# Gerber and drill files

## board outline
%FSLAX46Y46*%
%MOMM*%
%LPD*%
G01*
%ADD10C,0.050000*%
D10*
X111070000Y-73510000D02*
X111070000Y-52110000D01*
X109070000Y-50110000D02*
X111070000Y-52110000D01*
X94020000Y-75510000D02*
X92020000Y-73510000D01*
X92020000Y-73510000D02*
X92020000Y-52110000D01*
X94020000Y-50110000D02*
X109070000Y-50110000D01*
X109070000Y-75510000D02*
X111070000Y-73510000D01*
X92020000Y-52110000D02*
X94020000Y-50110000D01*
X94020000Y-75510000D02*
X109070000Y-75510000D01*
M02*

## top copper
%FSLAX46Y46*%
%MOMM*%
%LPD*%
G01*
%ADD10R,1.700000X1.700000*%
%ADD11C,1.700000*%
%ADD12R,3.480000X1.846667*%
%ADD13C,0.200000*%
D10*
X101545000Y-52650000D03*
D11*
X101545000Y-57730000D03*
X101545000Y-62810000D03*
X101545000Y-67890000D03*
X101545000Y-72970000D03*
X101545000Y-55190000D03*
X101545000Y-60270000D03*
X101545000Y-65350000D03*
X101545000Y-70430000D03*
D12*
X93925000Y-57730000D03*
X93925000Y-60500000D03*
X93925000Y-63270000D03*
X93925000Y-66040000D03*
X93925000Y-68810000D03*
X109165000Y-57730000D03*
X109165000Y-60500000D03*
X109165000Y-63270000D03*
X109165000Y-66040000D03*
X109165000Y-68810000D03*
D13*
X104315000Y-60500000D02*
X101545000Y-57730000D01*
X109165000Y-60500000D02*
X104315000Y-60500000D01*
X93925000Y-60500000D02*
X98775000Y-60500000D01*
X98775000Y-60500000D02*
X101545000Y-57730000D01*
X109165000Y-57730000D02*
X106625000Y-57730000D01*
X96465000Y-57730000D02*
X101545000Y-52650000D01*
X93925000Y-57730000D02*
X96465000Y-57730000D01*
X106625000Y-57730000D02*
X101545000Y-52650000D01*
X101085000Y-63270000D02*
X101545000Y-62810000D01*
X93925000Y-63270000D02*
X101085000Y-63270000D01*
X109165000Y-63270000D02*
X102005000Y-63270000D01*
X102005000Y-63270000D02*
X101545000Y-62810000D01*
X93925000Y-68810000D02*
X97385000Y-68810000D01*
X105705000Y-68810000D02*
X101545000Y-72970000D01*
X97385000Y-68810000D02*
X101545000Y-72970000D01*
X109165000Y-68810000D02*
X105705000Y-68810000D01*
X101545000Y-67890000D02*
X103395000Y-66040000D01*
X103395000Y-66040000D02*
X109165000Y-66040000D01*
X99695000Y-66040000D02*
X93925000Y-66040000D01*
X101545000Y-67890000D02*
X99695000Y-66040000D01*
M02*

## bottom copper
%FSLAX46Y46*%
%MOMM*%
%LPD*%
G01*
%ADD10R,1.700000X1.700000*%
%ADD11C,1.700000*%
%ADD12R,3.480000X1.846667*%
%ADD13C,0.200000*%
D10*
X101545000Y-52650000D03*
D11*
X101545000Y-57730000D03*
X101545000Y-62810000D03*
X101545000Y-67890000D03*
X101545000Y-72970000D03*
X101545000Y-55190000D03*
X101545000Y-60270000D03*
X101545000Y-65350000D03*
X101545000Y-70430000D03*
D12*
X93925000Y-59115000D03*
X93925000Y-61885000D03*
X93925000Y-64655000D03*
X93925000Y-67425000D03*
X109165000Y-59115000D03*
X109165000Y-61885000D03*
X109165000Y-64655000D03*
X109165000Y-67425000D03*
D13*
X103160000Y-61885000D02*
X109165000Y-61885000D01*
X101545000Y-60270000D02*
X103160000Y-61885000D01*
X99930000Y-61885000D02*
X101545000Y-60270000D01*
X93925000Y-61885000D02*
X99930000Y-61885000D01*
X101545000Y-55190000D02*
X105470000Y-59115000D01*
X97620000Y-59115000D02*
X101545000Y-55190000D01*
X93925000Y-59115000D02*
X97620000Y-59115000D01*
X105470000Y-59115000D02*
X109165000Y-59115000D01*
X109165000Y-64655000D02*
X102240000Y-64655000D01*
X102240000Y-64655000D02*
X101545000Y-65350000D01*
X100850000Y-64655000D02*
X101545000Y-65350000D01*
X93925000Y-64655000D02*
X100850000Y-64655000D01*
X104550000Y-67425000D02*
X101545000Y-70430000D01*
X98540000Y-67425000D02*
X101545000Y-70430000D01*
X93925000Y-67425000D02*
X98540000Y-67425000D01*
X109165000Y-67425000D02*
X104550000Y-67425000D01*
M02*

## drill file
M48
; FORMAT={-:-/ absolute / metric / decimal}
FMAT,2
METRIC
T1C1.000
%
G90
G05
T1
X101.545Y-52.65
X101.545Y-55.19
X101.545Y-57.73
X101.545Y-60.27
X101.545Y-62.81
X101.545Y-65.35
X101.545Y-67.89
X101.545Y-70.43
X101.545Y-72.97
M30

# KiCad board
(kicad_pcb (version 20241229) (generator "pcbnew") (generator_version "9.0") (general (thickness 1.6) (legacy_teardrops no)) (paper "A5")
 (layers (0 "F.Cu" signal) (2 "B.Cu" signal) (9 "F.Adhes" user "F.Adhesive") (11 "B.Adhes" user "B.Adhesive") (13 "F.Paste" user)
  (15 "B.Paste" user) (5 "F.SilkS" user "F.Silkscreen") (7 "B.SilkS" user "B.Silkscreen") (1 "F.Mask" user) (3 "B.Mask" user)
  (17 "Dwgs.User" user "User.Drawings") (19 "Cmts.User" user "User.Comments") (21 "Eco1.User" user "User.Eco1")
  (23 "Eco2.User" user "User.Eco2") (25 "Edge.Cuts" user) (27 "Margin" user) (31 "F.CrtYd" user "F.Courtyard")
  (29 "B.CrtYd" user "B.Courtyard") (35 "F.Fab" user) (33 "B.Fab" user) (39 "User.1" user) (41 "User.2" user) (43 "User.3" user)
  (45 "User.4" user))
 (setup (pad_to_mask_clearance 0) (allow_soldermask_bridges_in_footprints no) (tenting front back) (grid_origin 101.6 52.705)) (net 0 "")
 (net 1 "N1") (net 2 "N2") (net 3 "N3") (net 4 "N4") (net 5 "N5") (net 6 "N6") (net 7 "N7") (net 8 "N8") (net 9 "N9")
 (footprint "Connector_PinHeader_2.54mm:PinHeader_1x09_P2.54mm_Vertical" (layer "F.Cu") (at 101.545 72.97 180)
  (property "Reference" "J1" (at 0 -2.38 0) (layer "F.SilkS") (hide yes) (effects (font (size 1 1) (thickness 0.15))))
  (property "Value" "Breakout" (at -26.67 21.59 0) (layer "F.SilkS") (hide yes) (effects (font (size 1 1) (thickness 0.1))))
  (pad "1" thru_hole rect (at 0 20.32 180) (size 1.7 1.7) (drill 1) (layers "*.Cu" "*.Mask") (remove_unused_layers no) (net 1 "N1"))
  (pad "2" thru_hole circle (at 0 15.24 180) (size 1.7 1.7) (drill 1) (layers "*.Cu" "*.Mask") (remove_unused_layers no) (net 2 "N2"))
  (pad "3" thru_hole circle (at 0 10.16 180) (size 1.7 1.7) (drill 1) (layers "*.Cu" "*.Mask") (remove_unused_layers no) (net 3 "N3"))
  (pad "4" thru_hole circle (at 0 5.08 180) (size 1.7 1.7) (drill 1) (layers "*.Cu" "*.Mask") (remove_unused_layers no) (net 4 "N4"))
  (pad "5" thru_hole circle (at 0 0 180) (size 1.7 1.7) (drill 1) (layers "*.Cu" "*.Mask") (remove_unused_layers no) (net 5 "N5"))
  (pad "6" thru_hole circle (at 0 17.78 180) (size 1.7 1.7) (drill 1) (layers "*.Cu" "*.Mask") (remove_unused_layers no) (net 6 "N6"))
  (pad "7" thru_hole circle (at 0 12.7 180) (size 1.7 1.7) (drill 1) (layers "*.Cu" "*.Mask") (remove_unused_layers no) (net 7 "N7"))
  (pad "8" thru_hole circle (at 0 7.62 180) (size 1.7 1.7) (drill 1) (layers "*.Cu" "*.Mask") (remove_unused_layers no) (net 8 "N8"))
  (pad "9" thru_hole circle (at 0 2.54 180) (size 1.7 1.7) (drill 1) (layers "*.Cu" "*.Mask") (remove_unused_layers no) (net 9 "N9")))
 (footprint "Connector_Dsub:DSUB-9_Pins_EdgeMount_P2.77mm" (layer "F.Cu") (at 93.925 63.27 -90)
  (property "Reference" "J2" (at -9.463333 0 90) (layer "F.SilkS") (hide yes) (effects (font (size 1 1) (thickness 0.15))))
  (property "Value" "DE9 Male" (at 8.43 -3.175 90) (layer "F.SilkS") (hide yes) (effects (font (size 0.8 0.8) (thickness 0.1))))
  (pad "1" smd rect (at -5.54 0 270) (size 1.846667 3.48) (layers "F.Cu" "F.Mask" "F.Paste") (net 1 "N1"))
  (pad "2" smd rect (at -2.77 0 270) (size 1.846667 3.48) (layers "F.Cu" "F.Mask" "F.Paste") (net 2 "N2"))
  (pad "3" smd rect (at 0 0 270) (size 1.846667 3.48) (layers "F.Cu" "F.Mask" "F.Paste") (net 3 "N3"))
  (pad "4" smd rect (at 2.77 0 270) (size 1.846667 3.48) (layers "F.Cu" "F.Mask" "F.Paste") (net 4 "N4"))
  (pad "5" smd rect (at 5.54 0 270) (size 1.846667 3.48) (layers "F.Cu" "F.Mask" "F.Paste") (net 5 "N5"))
  (pad "6" smd rect (at -4.155 0 270) (size 1.846667 3.48) (layers "B.Cu" "B.Mask" "B.Paste") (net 6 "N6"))
  (pad "7" smd rect (at -1.385 0 270) (size 1.846667 3.48) (layers "B.Cu" "B.Mask" "B.Paste") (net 7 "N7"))
  (pad "8" smd rect (at 1.385 0 270) (size 1.846667 3.48) (layers "B.Cu" "B.Mask" "B.Paste") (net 8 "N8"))
  (pad "9" smd rect (at 4.155 0 270) (size 1.846667 3.48) (layers "B.Cu" "B.Mask" "B.Paste") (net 9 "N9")))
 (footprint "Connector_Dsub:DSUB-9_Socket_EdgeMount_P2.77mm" (layer "F.Cu") (at 109.165 63.27 90)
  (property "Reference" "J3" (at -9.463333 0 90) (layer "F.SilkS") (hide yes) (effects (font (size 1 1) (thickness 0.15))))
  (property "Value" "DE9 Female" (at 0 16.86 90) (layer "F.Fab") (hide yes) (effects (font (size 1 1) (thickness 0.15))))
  (pad "1" smd rect (at 5.54 0 90) (size 1.846667 3.48) (layers "F.Cu" "F.Mask" "F.Paste") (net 1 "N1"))
  (pad "2" smd rect (at 2.77 0 90) (size 1.846667 3.48) (layers "F.Cu" "F.Mask" "F.Paste") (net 2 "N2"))
  (pad "3" smd rect (at 0 0 90) (size 1.846667 3.48) (layers "F.Cu" "F.Mask" "F.Paste") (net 3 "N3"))
  (pad "4" smd rect (at -2.77 0 90) (size 1.846667 3.48) (layers "F.Cu" "F.Mask" "F.Paste") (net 4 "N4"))
  (pad "5" smd rect (at -5.54 0 90) (size 1.846667 3.48) (layers "F.Cu" "F.Mask" "F.Paste") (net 5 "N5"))
  (pad "6" smd rect (at 4.155 0 90) (size 1.846667 3.48) (layers "B.Cu" "B.Mask" "B.Paste") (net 6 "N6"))
  (pad "7" smd rect (at 1.385 0 90) (size 1.846667 3.48) (layers "B.Cu" "B.Mask" "B.Paste") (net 7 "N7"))
  (pad "8" smd rect (at -1.385 0 90) (size 1.846667 3.48) (layers "B.Cu" "B.Mask" "B.Paste") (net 8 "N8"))
  (pad "9" smd rect (at -4.155 0 90) (size 1.846667 3.48) (layers "B.Cu" "B.Mask" "B.Paste") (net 9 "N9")))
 (gr_line (start 111.07 73.51) (end 111.07 52.11) (stroke (width 0.05) (type default)) (layer "Edge.Cuts"))
 (gr_line (start 109.07 50.11) (end 111.07 52.11) (stroke (width 0.05) (type default)) (layer "Edge.Cuts"))
 (gr_line (start 94.02 75.51) (end 92.02 73.51) (stroke (width 0.05) (type default)) (layer "Edge.Cuts"))
 (gr_line (start 92.02 73.51) (end 92.02 52.11) (stroke (width 0.05) (type default)) (layer "Edge.Cuts"))
 (gr_line (start 94.02 50.11) (end 109.07 50.11) (stroke (width 0.05) (type default)) (layer "Edge.Cuts"))
 (gr_line (start 109.07 75.51) (end 111.07 73.51) (stroke (width 0.05) (type default)) (layer "Edge.Cuts"))
 (gr_line (start 92.02 52.11) (end 94.02 50.11) (stroke (width 0.05) (type default)) (layer "Edge.Cuts"))
 (gr_line (start 94.02 75.51) (end 109.07 75.51) (stroke (width 0.05) (type default)) (layer "Edge.Cuts"))
 (segment (start 103.16 61.885) (end 109.165 61.885) (width 0.2) (layer "B.Cu") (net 7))
 (segment (start 101.545 60.27) (end 103.16 61.885) (width 0.2) (layer "B.Cu") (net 7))
 (segment (start 99.93 61.885) (end 101.545 60.27) (width 0.2) (layer "B.Cu") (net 7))
 (segment (start 93.925 61.885) (end 99.93 61.885) (width 0.2) (layer "B.Cu") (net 7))
 (segment (start 101.545 55.19) (end 105.47 59.115) (width 0.2) (layer "B.Cu") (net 6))
 (segment (start 97.62 59.115) (end 101.545 55.19) (width 0.2) (layer "B.Cu") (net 6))
 (segment (start 93.925 59.115) (end 97.62 59.115) (width 0.2) (layer "B.Cu") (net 6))
 (segment (start 105.47 59.115) (end 109.165 59.115) (width 0.2) (layer "B.Cu") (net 6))
 (segment (start 104.315 60.5) (end 101.545 57.73) (width 0.2) (layer "F.Cu") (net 2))
 (segment (start 109.165 60.5) (end 104.315 60.5) (width 0.2) (layer "F.Cu") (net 2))
 (segment (start 93.925 60.5) (end 98.775 60.5) (width 0.2) (layer "F.Cu") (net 2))
 (segment (start 98.775 60.5) (end 101.545 57.73) (width 0.2) (layer "F.Cu") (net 2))
 (segment (start 109.165 57.73) (end 106.625 57.73) (width 0.2) (layer "F.Cu") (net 1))
 (segment (start 96.465 57.73) (end 101.545 52.65) (width 0.2) (layer "F.Cu") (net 1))
 (segment (start 93.925 57.73) (end 96.465 57.73) (width 0.2) (layer "F.Cu") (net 1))
 (segment (start 106.625 57.73) (end 101.545 52.65) (width 0.2) (layer "F.Cu") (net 1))
 (segment (start 109.165 64.655) (end 102.24 64.655) (width 0.2) (layer "B.Cu") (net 8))
 (segment (start 102.24 64.655) (end 101.545 65.35) (width 0.2) (layer "B.Cu") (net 8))
 (segment (start 100.85 64.655) (end 101.545 65.35) (width 0.2) (layer "B.Cu") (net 8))
 (segment (start 93.925 64.655) (end 100.85 64.655) (width 0.2) (layer "B.Cu") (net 8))
 (segment (start 101.085 63.27) (end 101.545 62.81) (width 0.2) (layer "F.Cu") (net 3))
 (segment (start 93.925 63.27) (end 101.085 63.27) (width 0.2) (layer "F.Cu") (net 3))
 (segment (start 109.165 63.27) (end 102.005 63.27) (width 0.2) (layer "F.Cu") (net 3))
 (segment (start 102.005 63.27) (end 101.545 62.81) (width 0.2) (layer "F.Cu") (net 3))
 (segment (start 93.925 68.81) (end 97.385 68.81) (width 0.2) (layer "F.Cu") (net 5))
 (segment (start 105.705 68.81) (end 101.545 72.97) (width 0.2) (layer "F.Cu") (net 5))
 (segment (start 97.385 68.81) (end 101.545 72.97) (width 0.2) (layer "F.Cu") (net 5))
 (segment (start 109.165 68.81) (end 105.705 68.81) (width 0.2) (layer "F.Cu") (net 5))
 (segment (start 101.545 67.89) (end 103.395 66.04) (width 0.2) (layer "F.Cu") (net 4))
 (segment (start 103.395 66.04) (end 109.165 66.04) (width 0.2) (layer "F.Cu") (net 4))
 (segment (start 99.695 66.04) (end 93.925 66.04) (width 0.2) (layer "F.Cu") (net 4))
 (segment (start 101.545 67.89) (end 99.695 66.04) (width 0.2) (layer "F.Cu") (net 4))
 (segment (start 104.55 67.425) (end 101.545 70.43) (width 0.2) (layer "B.Cu") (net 9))
 (segment (start 98.54 67.425) (end 101.545 70.43) (width 0.2) (layer "B.Cu") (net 9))
 (segment (start 93.925 67.425) (end 98.54 67.425) (width 0.2) (layer "B.Cu") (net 9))
 (segment (start 109.165 67.425) (end 104.55 67.425) (width 0.2) (layer "B.Cu") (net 9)))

